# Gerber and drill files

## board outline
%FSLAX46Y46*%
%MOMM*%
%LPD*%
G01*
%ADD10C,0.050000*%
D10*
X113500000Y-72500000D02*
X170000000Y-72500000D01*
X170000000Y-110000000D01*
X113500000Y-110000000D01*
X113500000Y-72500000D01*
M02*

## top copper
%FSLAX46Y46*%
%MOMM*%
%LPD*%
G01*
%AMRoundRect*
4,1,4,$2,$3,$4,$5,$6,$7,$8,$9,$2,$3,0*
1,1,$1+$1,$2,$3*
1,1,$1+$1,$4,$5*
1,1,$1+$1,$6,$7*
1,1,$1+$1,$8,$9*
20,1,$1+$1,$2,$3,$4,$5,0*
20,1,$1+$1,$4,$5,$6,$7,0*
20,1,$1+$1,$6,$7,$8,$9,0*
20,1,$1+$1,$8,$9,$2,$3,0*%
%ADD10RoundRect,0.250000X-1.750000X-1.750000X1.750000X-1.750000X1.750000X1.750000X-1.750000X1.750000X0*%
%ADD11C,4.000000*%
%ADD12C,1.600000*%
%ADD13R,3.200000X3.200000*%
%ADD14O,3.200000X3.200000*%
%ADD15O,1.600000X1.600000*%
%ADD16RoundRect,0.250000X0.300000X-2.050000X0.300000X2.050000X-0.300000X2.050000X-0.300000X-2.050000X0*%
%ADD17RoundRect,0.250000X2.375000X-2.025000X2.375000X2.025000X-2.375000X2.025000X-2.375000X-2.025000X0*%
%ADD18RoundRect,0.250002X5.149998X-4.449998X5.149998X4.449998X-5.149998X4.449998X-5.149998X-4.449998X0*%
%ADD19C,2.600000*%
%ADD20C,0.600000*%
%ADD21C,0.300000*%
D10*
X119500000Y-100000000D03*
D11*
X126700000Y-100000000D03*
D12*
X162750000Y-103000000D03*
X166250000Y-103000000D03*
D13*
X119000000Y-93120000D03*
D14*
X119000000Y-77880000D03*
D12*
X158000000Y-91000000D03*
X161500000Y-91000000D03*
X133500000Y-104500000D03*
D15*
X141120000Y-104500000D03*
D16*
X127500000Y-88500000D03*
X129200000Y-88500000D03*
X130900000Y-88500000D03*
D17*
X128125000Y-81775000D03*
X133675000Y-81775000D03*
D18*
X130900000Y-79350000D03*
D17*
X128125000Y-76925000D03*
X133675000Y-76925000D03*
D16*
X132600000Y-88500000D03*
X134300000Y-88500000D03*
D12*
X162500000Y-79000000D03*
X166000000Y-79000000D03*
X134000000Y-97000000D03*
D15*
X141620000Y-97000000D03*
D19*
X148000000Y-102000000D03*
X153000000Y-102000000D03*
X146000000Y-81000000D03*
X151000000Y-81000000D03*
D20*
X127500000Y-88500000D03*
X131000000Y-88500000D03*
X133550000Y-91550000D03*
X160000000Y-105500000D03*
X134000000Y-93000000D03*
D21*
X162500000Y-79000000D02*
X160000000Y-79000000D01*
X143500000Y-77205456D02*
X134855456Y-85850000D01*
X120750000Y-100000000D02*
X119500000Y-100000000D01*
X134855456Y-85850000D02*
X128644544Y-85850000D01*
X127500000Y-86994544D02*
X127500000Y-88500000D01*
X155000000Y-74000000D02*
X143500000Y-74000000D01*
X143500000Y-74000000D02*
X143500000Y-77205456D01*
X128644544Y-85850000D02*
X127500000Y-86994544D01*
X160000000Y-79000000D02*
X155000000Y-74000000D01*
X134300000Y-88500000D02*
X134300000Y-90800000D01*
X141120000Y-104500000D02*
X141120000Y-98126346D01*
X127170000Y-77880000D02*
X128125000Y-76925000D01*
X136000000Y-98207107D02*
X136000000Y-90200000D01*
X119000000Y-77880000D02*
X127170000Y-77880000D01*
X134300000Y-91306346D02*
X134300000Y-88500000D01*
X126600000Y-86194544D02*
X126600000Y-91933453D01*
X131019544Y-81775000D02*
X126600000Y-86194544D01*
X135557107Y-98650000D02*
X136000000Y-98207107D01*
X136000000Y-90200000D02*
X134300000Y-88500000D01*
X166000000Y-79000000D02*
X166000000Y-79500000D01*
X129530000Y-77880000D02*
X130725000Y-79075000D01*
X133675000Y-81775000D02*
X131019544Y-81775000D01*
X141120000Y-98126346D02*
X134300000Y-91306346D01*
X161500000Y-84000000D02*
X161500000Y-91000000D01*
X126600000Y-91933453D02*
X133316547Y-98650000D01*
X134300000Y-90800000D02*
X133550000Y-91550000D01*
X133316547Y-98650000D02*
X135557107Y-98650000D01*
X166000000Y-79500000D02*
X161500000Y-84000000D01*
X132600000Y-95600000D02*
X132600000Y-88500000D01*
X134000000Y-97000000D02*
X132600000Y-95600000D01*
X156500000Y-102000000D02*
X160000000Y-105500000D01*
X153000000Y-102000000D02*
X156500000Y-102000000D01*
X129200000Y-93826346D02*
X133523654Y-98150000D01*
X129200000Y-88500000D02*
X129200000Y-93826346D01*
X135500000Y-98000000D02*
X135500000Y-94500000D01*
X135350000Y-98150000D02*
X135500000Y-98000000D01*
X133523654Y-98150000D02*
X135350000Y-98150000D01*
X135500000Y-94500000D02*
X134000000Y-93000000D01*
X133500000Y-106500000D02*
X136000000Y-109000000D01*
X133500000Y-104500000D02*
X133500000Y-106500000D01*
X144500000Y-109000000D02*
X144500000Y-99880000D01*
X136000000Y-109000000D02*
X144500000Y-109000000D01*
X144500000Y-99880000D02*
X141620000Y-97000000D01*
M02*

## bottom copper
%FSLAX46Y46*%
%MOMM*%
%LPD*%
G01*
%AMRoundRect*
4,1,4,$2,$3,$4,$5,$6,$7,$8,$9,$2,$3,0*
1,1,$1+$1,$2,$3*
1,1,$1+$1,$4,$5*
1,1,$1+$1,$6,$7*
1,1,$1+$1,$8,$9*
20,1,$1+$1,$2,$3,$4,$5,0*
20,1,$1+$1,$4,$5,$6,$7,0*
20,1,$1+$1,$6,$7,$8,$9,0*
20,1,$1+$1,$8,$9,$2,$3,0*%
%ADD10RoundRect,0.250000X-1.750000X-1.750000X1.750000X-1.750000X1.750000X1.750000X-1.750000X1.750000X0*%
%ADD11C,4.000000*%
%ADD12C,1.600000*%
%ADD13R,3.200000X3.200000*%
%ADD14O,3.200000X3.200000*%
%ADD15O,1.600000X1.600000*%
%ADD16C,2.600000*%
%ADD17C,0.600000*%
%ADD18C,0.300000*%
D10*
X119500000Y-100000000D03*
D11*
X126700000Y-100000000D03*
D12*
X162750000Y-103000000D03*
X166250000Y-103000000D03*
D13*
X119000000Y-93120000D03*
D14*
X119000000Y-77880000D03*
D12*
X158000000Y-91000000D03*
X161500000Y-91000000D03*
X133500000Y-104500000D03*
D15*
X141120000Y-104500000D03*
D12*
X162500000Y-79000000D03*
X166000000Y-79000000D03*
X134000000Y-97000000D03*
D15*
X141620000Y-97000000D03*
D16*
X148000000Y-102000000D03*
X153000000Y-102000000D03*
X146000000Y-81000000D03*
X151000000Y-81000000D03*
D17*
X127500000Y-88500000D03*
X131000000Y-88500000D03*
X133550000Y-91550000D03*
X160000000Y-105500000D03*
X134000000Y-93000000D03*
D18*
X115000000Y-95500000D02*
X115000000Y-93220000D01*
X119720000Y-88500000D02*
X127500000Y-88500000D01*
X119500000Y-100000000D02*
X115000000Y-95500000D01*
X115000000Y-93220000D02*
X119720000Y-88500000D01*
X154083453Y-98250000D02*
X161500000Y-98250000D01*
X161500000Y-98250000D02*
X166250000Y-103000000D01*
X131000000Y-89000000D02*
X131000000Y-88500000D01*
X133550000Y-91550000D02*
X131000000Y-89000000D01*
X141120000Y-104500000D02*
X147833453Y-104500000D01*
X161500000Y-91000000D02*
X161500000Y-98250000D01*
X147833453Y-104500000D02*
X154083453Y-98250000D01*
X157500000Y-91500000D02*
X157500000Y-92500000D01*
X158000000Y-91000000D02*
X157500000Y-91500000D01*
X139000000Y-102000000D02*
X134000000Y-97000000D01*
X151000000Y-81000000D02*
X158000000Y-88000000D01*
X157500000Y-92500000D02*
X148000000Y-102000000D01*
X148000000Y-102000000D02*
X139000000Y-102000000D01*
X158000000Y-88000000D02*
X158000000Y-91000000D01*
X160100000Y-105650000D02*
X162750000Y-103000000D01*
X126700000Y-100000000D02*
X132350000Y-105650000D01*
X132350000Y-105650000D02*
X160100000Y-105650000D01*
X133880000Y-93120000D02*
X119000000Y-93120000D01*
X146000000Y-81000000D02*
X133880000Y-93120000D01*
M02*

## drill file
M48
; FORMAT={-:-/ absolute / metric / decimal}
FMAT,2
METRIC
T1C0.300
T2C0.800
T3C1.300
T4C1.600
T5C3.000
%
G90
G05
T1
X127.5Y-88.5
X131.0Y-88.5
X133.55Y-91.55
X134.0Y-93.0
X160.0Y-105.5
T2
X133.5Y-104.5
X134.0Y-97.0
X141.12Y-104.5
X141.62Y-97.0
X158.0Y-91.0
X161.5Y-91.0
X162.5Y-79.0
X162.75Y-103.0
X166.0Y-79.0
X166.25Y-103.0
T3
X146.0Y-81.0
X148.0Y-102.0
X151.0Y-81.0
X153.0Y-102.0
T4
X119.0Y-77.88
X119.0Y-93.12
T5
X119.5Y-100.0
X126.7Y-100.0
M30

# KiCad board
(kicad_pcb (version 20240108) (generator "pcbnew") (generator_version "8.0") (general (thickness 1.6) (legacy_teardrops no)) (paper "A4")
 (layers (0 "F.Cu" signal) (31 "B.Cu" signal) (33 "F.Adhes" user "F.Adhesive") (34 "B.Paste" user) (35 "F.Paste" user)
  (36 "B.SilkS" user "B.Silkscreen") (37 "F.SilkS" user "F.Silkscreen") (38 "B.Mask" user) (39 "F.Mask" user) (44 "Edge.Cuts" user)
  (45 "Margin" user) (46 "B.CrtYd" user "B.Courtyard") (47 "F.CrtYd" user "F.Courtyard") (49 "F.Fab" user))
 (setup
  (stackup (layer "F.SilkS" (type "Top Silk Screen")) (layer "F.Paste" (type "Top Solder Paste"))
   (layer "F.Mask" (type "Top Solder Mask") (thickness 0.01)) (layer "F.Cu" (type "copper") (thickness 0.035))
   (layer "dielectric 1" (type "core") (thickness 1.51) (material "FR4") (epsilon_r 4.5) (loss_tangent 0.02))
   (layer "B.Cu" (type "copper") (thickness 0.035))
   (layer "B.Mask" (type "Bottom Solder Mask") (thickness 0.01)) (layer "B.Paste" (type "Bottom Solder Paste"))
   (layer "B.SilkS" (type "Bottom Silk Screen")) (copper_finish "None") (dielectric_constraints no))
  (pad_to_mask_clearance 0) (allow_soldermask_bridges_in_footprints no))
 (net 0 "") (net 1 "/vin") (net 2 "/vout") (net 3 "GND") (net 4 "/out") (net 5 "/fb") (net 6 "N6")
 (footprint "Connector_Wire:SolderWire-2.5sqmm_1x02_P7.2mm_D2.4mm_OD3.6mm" (layer "F.Cu") (at 119.5 100)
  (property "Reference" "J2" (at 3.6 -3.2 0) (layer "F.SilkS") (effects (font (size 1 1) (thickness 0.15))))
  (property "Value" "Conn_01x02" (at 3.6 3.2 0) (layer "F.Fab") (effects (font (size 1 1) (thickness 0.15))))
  (pad "1" thru_hole roundrect (at 0 0) (size 4 4) (drill 3) (layers "*.Cu" "*.Mask") (remove_unused_layers no) (roundrect_rratio 0.0625)
   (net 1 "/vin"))
  (pad "2" thru_hole circle (at 7.2 0) (size 4 4) (drill 3) (layers "*.Cu" "*.Mask") (remove_unused_layers no) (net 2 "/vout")))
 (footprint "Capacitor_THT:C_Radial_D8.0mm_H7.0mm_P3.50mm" (layer "F.Cu") (at 162.75 103)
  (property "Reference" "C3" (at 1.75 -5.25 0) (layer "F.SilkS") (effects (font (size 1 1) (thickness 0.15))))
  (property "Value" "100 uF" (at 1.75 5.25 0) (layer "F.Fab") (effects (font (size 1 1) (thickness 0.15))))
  (pad "1" thru_hole circle (at 0 0) (size 1.6 1.6) (drill 0.8) (layers "*.Cu" "*.Mask") (remove_unused_layers no) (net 2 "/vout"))
  (pad "2" thru_hole circle (at 3.5 0) (size 1.6 1.6) (drill 0.8) (layers "*.Cu" "*.Mask") (remove_unused_layers no) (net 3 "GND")))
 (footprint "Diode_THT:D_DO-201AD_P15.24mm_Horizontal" (layer "F.Cu") (at 119 93.12 90)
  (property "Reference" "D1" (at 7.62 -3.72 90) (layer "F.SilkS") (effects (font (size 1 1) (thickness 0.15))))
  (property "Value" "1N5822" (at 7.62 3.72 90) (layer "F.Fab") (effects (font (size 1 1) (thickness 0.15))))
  (pad "1" thru_hole rect (at 0 0 90) (size 3.2 3.2) (drill 1.6) (layers "*.Cu" "*.Mask") (remove_unused_layers no) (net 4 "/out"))
  (pad "2" thru_hole oval (at 15.24 0 90) (size 3.2 3.2) (drill 1.6) (layers "*.Cu" "*.Mask") (remove_unused_layers no) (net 3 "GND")))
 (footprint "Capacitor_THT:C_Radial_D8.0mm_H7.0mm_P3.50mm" (layer "F.Cu") (at 158 91)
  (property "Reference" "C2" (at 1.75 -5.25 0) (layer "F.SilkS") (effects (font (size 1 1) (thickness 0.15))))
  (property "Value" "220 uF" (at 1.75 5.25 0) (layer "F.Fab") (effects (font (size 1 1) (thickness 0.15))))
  (pad "1" thru_hole circle (at 0 0) (size 1.6 1.6) (drill 0.8) (layers "*.Cu" "*.Mask") (remove_unused_layers no) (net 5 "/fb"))
  (pad "2" thru_hole circle (at 3.5 0) (size 1.6 1.6) (drill 0.8) (layers "*.Cu" "*.Mask") (remove_unused_layers no) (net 3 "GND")))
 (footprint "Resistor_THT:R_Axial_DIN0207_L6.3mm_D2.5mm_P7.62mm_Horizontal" (layer "F.Cu") (at 133.5 104.5)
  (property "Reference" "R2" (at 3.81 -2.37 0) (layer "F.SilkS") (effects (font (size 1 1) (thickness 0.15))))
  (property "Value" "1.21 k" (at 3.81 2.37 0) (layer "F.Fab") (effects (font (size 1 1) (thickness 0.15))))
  (pad "1" thru_hole circle (at 0 0) (size 1.6 1.6) (drill 0.8) (layers "*.Cu" "*.Mask") (remove_unused_layers no) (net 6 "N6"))
  (pad "2" thru_hole oval (at 7.62 0) (size 1.6 1.6) (drill 0.8) (layers "*.Cu" "*.Mask") (remove_unused_layers no) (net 3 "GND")))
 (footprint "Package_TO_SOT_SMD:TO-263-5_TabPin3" (layer "F.Cu") (at 130.9 80.85 90)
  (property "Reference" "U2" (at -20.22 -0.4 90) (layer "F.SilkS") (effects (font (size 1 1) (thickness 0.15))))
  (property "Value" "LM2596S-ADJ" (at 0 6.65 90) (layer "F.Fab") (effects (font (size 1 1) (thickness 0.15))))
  (pad "1" smd roundrect (at -7.65 -3.4 90) (size 4.6 1.1) (layers "F.Cu" "F.Paste" "F.Mask") (roundrect_rratio 0.227273) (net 1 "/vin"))
  (pad "2" smd roundrect (at -7.65 -1.7 90) (size 4.6 1.1) (layers "F.Cu" "F.Paste" "F.Mask") (roundrect_rratio 0.227273) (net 4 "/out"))
  (pad "3" smd roundrect (at -7.65 0 90) (size 4.6 1.1) (layers "F.Cu" "F.Paste" "F.Mask") (roundrect_rratio 0.227273) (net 3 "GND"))
  (pad "3" smd roundrect (at -0.925 -2.775 90) (size 4.55 5.25) (layers "F.Cu" "F.Paste") (roundrect_rratio 0.054945) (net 3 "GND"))
  (pad "3" smd roundrect (at -0.925 2.775 90) (size 4.55 5.25) (layers "F.Cu" "F.Paste") (roundrect_rratio 0.054945) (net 3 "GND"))
  (pad "3" smd roundrect (at 1.5 0 90) (size 9.4 10.8) (layers "F.Cu" "F.Mask") (roundrect_rratio 0.026596) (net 3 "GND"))
  (pad "3" smd roundrect (at 3.925 -2.775 90) (size 4.55 5.25) (layers "F.Cu" "F.Paste") (roundrect_rratio 0.054945) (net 3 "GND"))
  (pad "3" smd roundrect (at 3.925 2.775 90) (size 4.55 5.25) (layers "F.Cu" "F.Paste") (roundrect_rratio 0.054945) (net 3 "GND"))
  (pad "4" smd roundrect (at -7.65 1.7 90) (size 4.6 1.1) (layers "F.Cu" "F.Paste" "F.Mask") (roundrect_rratio 0.227273) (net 5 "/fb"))
  (pad "5" smd roundrect (at -7.65 3.4 90) (size 4.6 1.1) (layers "F.Cu" "F.Paste" "F.Mask") (roundrect_rratio 0.227273) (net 3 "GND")))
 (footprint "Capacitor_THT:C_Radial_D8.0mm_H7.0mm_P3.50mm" (layer "F.Cu") (at 162.5 79)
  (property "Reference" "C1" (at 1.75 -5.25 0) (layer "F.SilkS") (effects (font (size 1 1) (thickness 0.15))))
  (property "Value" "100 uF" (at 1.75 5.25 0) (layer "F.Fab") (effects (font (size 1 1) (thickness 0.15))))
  (pad "1" thru_hole circle (at 0 0) (size 1.6 1.6) (drill 0.8) (layers "*.Cu" "*.Mask") (remove_unused_layers no) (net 1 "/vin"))
  (pad "2" thru_hole circle (at 3.5 0) (size 1.6 1.6) (drill 0.8) (layers "*.Cu" "*.Mask") (remove_unused_layers no) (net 3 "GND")))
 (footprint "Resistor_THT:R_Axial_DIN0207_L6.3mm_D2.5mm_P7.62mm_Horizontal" (layer "F.Cu") (at 134 97)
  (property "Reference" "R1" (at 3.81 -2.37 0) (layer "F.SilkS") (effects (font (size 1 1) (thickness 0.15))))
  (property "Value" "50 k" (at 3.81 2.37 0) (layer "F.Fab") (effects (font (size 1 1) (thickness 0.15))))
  (pad "1" thru_hole circle (at 0 0) (size 1.6 1.6) (drill 0.8) (layers "*.Cu" "*.Mask") (remove_unused_layers no) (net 5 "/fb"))
  (pad "2" thru_hole oval (at 7.62 0) (size 1.6 1.6) (drill 0.8) (layers "*.Cu" "*.Mask") (remove_unused_layers no) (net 6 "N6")))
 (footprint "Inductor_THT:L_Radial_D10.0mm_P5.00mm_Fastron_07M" (layer "F.Cu") (at 148 102)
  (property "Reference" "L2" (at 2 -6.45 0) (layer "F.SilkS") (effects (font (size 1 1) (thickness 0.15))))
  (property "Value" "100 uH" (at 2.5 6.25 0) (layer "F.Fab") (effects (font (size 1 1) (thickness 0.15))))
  (pad "1" thru_hole circle (at 0 0) (size 2.6 2.6) (drill 1.3) (layers "*.Cu" "*.Mask") (remove_unused_layers no) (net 5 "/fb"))
  (pad "2" thru_hole circle (at 5 0) (size 2.6 2.6) (drill 1.3) (layers "*.Cu" "*.Mask") (remove_unused_layers no) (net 2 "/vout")))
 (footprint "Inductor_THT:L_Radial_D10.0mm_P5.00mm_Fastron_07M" (layer "F.Cu") (at 146 81)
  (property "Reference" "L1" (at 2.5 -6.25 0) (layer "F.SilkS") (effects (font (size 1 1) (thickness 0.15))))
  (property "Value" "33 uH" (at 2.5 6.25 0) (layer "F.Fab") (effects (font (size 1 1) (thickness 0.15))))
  (pad "1" thru_hole circle (at 0 0) (size 2.6 2.6) (drill 1.3) (layers "*.Cu" "*.Mask") (remove_unused_layers no) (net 4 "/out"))
  (pad "2" thru_hole circle (at 5 0) (size 2.6 2.6) (drill 1.3) (layers "*.Cu" "*.Mask") (remove_unused_layers no) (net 5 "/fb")))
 (gr_rect (start 113.5 72.5) (end 170 110) (stroke (width 0.05) (type default)) (fill none) (layer "Edge.Cuts"))
 (segment (start 162.5 79) (end 160 79) (width 0.3) (layer "F.Cu") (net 1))
 (segment (start 143.5 77.205456) (end 134.855456 85.85) (width 0.3) (layer "F.Cu") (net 1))
 (segment (start 120.75 100) (end 119.5 100) (width 0.3) (layer "F.Cu") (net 1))
 (segment (start 134.855456 85.85) (end 128.644544 85.85) (width 0.3) (layer "F.Cu") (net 1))
 (segment (start 127.5 86.994544) (end 127.5 88.5) (width 0.3) (layer "F.Cu") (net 1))
 (segment (start 155 74) (end 143.5 74) (width 0.3) (layer "F.Cu") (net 1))
 (segment (start 143.5 74) (end 143.5 77.205456) (width 0.3) (layer "F.Cu") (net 1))
 (segment (start 128.644544 85.85) (end 127.5 86.994544) (width 0.3) (layer "F.Cu") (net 1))
 (segment (start 160 79) (end 155 74) (width 0.3) (layer "F.Cu") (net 1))
 (via (at 127.5 88.5) (size 0.6) (drill 0.3) (layers "F.Cu" "B.Cu") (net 1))
 (segment (start 115 95.5) (end 115 93.22) (width 0.3) (layer "B.Cu") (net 1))
 (segment (start 119.72 88.5) (end 127.5 88.5) (width 0.3) (layer "B.Cu") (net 1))
 (segment (start 119.5 100) (end 115 95.5) (width 0.3) (layer "B.Cu") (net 1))
 (segment (start 115 93.22) (end 119.72 88.5) (width 0.3) (layer "B.Cu") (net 1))
 (segment (start 134.3 88.5) (end 134.3 90.8) (width 0.3) (layer "F.Cu") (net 3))
 (segment (start 141.12 104.5) (end 141.12 98.126346) (width 0.3) (layer "F.Cu") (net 3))
 (segment (start 127.17 77.88) (end 128.125 76.925) (width 0.3) (layer "F.Cu") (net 3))
 (segment (start 136 98.207107) (end 136 90.2) (width 0.3) (layer "F.Cu") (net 3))
 (segment (start 119 77.88) (end 127.17 77.88) (width 0.3) (layer "F.Cu") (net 3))
 (segment (start 134.3 91.306346) (end 134.3 88.5) (width 0.3) (layer "F.Cu") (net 3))
 (segment (start 126.6 86.194544) (end 126.6 91.933453) (width 0.3) (layer "F.Cu") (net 3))
 (segment (start 131.019544 81.775) (end 126.6 86.194544) (width 0.3) (layer "F.Cu") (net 3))
 (segment (start 135.557107 98.65) (end 136 98.207107) (width 0.3) (layer "F.Cu") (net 3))
 (segment (start 136 90.2) (end 134.3 88.5) (width 0.3) (layer "F.Cu") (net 3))
 (segment (start 166 79) (end 166 79.5) (width 0.3) (layer "F.Cu") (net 3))
 (segment (start 129.53 77.88) (end 130.725 79.075) (width 0.3) (layer "F.Cu") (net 3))
 (segment (start 133.675 81.775) (end 131.019544 81.775) (width 0.3) (layer "F.Cu") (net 3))
 (segment (start 141.12 98.126346) (end 134.3 91.306346) (width 0.3) (layer "F.Cu") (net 3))
 (segment (start 161.5 84) (end 161.5 91) (width 0.3) (layer "F.Cu") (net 3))
 (segment (start 126.6 91.933453) (end 133.316547 98.65) (width 0.3) (layer "F.Cu") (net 3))
 (segment (start 134.3 90.8) (end 133.55 91.55) (width 0.3) (layer "F.Cu") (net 3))
 (segment (start 133.316547 98.65) (end 135.557107 98.65) (width 0.3) (layer "F.Cu") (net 3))
 (segment (start 166 79.5) (end 161.5 84) (width 0.3) (layer "F.Cu") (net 3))
 (via (at 131 88.5) (size 0.6) (drill 0.3) (layers "F.Cu" "B.Cu") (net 3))
 (via (at 133.55 91.55) (size 0.6) (drill 0.3) (layers "F.Cu" "B.Cu") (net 3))
 (segment (start 154.083453 98.25) (end 161.5 98.25) (width 0.3) (layer "B.Cu") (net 3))
 (segment (start 161.5 98.25) (end 166.25 103) (width 0.3) (layer "B.Cu") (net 3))
 (segment (start 131 89) (end 131 88.5) (width 0.3) (layer "B.Cu") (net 3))
 (segment (start 133.55 91.55) (end 131 89) (width 0.3) (layer "B.Cu") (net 3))
 (segment (start 141.12 104.5) (end 147.833453 104.5) (width 0.3) (layer "B.Cu") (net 3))
 (segment (start 161.5 91) (end 161.5 98.25) (width 0.3) (layer "B.Cu") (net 3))
 (segment (start 147.833453 104.5) (end 154.083453 98.25) (width 0.3) (layer "B.Cu") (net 3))
 (segment (start 132.6 95.6) (end 132.6 88.5) (width 0.3) (layer "F.Cu") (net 5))
 (segment (start 134 97) (end 132.6 95.6) (width 0.3) (layer "F.Cu") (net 5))
 (segment (start 157.5 91.5) (end 157.5 92.5) (width 0.3) (layer "B.Cu") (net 5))
 (segment (start 158 91) (end 157.5 91.5) (width 0.3) (layer "B.Cu") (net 5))
 (segment (start 139 102) (end 134 97) (width 0.3) (layer "B.Cu") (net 5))
 (segment (start 151 81) (end 158 88) (width 0.3) (layer "B.Cu") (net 5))
 (segment (start 157.5 92.5) (end 148 102) (width 0.3) (layer "B.Cu") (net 5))
 (segment (start 148 102) (end 139 102) (width 0.3) (layer "B.Cu") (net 5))
 (segment (start 158 88) (end 158 91) (width 0.3) (layer "B.Cu") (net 5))
 (segment (start 156.5 102) (end 160 105.5) (width 0.3) (layer "F.Cu") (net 2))
 (segment (start 153 102) (end 156.5 102) (width 0.3) (layer "F.Cu") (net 2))
 (via (at 160 105.5) (size 0.6) (drill 0.3) (layers "F.Cu" "B.Cu") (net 2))
 (segment (start 160.1 105.65) (end 162.75 103) (width 0.3) (layer "B.Cu") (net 2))
 (segment (start 126.7 100) (end 132.35 105.65) (width 0.3) (layer "B.Cu") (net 2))
 (segment (start 132.35 105.65) (end 160.1 105.65) (width 0.3) (layer "B.Cu") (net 2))
 (segment (start 129.2 93.826346) (end 133.523654 98.15) (width 0.3) (layer "F.Cu") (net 4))
 (segment (start 129.2 88.5) (end 129.2 93.826346) (width 0.3) (layer "F.Cu") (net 4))
 (segment (start 135.5 98) (end 135.5 94.5) (width 0.3) (layer "F.Cu") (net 4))
 (segment (start 135.35 98.15) (end 135.5 98) (width 0.3) (layer "F.Cu") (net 4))
 (segment (start 133.523654 98.15) (end 135.35 98.15) (width 0.3) (layer "F.Cu") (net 4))
 (segment (start 135.5 94.5) (end 134 93) (width 0.3) (layer "F.Cu") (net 4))
 (via (at 134 93) (size 0.6) (drill 0.3) (layers "F.Cu" "B.Cu") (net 4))
 (segment (start 133.88 93.12) (end 119 93.12) (width 0.3) (layer "B.Cu") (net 4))
 (segment (start 146 81) (end 133.88 93.12) (width 0.3) (layer "B.Cu") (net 4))
 (segment (start 133.5 106.5) (end 136 109) (width 0.3) (layer "F.Cu") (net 6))
 (segment (start 133.5 104.5) (end 133.5 106.5) (width 0.3) (layer "F.Cu") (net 6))
 (segment (start 144.5 109) (end 144.5 99.88) (width 0.3) (layer "F.Cu") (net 6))
 (segment (start 136 109) (end 144.5 109) (width 0.3) (layer "F.Cu") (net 6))
 (segment (start 144.5 99.88) (end 141.62 97) (width 0.3) (layer "F.Cu") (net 6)))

